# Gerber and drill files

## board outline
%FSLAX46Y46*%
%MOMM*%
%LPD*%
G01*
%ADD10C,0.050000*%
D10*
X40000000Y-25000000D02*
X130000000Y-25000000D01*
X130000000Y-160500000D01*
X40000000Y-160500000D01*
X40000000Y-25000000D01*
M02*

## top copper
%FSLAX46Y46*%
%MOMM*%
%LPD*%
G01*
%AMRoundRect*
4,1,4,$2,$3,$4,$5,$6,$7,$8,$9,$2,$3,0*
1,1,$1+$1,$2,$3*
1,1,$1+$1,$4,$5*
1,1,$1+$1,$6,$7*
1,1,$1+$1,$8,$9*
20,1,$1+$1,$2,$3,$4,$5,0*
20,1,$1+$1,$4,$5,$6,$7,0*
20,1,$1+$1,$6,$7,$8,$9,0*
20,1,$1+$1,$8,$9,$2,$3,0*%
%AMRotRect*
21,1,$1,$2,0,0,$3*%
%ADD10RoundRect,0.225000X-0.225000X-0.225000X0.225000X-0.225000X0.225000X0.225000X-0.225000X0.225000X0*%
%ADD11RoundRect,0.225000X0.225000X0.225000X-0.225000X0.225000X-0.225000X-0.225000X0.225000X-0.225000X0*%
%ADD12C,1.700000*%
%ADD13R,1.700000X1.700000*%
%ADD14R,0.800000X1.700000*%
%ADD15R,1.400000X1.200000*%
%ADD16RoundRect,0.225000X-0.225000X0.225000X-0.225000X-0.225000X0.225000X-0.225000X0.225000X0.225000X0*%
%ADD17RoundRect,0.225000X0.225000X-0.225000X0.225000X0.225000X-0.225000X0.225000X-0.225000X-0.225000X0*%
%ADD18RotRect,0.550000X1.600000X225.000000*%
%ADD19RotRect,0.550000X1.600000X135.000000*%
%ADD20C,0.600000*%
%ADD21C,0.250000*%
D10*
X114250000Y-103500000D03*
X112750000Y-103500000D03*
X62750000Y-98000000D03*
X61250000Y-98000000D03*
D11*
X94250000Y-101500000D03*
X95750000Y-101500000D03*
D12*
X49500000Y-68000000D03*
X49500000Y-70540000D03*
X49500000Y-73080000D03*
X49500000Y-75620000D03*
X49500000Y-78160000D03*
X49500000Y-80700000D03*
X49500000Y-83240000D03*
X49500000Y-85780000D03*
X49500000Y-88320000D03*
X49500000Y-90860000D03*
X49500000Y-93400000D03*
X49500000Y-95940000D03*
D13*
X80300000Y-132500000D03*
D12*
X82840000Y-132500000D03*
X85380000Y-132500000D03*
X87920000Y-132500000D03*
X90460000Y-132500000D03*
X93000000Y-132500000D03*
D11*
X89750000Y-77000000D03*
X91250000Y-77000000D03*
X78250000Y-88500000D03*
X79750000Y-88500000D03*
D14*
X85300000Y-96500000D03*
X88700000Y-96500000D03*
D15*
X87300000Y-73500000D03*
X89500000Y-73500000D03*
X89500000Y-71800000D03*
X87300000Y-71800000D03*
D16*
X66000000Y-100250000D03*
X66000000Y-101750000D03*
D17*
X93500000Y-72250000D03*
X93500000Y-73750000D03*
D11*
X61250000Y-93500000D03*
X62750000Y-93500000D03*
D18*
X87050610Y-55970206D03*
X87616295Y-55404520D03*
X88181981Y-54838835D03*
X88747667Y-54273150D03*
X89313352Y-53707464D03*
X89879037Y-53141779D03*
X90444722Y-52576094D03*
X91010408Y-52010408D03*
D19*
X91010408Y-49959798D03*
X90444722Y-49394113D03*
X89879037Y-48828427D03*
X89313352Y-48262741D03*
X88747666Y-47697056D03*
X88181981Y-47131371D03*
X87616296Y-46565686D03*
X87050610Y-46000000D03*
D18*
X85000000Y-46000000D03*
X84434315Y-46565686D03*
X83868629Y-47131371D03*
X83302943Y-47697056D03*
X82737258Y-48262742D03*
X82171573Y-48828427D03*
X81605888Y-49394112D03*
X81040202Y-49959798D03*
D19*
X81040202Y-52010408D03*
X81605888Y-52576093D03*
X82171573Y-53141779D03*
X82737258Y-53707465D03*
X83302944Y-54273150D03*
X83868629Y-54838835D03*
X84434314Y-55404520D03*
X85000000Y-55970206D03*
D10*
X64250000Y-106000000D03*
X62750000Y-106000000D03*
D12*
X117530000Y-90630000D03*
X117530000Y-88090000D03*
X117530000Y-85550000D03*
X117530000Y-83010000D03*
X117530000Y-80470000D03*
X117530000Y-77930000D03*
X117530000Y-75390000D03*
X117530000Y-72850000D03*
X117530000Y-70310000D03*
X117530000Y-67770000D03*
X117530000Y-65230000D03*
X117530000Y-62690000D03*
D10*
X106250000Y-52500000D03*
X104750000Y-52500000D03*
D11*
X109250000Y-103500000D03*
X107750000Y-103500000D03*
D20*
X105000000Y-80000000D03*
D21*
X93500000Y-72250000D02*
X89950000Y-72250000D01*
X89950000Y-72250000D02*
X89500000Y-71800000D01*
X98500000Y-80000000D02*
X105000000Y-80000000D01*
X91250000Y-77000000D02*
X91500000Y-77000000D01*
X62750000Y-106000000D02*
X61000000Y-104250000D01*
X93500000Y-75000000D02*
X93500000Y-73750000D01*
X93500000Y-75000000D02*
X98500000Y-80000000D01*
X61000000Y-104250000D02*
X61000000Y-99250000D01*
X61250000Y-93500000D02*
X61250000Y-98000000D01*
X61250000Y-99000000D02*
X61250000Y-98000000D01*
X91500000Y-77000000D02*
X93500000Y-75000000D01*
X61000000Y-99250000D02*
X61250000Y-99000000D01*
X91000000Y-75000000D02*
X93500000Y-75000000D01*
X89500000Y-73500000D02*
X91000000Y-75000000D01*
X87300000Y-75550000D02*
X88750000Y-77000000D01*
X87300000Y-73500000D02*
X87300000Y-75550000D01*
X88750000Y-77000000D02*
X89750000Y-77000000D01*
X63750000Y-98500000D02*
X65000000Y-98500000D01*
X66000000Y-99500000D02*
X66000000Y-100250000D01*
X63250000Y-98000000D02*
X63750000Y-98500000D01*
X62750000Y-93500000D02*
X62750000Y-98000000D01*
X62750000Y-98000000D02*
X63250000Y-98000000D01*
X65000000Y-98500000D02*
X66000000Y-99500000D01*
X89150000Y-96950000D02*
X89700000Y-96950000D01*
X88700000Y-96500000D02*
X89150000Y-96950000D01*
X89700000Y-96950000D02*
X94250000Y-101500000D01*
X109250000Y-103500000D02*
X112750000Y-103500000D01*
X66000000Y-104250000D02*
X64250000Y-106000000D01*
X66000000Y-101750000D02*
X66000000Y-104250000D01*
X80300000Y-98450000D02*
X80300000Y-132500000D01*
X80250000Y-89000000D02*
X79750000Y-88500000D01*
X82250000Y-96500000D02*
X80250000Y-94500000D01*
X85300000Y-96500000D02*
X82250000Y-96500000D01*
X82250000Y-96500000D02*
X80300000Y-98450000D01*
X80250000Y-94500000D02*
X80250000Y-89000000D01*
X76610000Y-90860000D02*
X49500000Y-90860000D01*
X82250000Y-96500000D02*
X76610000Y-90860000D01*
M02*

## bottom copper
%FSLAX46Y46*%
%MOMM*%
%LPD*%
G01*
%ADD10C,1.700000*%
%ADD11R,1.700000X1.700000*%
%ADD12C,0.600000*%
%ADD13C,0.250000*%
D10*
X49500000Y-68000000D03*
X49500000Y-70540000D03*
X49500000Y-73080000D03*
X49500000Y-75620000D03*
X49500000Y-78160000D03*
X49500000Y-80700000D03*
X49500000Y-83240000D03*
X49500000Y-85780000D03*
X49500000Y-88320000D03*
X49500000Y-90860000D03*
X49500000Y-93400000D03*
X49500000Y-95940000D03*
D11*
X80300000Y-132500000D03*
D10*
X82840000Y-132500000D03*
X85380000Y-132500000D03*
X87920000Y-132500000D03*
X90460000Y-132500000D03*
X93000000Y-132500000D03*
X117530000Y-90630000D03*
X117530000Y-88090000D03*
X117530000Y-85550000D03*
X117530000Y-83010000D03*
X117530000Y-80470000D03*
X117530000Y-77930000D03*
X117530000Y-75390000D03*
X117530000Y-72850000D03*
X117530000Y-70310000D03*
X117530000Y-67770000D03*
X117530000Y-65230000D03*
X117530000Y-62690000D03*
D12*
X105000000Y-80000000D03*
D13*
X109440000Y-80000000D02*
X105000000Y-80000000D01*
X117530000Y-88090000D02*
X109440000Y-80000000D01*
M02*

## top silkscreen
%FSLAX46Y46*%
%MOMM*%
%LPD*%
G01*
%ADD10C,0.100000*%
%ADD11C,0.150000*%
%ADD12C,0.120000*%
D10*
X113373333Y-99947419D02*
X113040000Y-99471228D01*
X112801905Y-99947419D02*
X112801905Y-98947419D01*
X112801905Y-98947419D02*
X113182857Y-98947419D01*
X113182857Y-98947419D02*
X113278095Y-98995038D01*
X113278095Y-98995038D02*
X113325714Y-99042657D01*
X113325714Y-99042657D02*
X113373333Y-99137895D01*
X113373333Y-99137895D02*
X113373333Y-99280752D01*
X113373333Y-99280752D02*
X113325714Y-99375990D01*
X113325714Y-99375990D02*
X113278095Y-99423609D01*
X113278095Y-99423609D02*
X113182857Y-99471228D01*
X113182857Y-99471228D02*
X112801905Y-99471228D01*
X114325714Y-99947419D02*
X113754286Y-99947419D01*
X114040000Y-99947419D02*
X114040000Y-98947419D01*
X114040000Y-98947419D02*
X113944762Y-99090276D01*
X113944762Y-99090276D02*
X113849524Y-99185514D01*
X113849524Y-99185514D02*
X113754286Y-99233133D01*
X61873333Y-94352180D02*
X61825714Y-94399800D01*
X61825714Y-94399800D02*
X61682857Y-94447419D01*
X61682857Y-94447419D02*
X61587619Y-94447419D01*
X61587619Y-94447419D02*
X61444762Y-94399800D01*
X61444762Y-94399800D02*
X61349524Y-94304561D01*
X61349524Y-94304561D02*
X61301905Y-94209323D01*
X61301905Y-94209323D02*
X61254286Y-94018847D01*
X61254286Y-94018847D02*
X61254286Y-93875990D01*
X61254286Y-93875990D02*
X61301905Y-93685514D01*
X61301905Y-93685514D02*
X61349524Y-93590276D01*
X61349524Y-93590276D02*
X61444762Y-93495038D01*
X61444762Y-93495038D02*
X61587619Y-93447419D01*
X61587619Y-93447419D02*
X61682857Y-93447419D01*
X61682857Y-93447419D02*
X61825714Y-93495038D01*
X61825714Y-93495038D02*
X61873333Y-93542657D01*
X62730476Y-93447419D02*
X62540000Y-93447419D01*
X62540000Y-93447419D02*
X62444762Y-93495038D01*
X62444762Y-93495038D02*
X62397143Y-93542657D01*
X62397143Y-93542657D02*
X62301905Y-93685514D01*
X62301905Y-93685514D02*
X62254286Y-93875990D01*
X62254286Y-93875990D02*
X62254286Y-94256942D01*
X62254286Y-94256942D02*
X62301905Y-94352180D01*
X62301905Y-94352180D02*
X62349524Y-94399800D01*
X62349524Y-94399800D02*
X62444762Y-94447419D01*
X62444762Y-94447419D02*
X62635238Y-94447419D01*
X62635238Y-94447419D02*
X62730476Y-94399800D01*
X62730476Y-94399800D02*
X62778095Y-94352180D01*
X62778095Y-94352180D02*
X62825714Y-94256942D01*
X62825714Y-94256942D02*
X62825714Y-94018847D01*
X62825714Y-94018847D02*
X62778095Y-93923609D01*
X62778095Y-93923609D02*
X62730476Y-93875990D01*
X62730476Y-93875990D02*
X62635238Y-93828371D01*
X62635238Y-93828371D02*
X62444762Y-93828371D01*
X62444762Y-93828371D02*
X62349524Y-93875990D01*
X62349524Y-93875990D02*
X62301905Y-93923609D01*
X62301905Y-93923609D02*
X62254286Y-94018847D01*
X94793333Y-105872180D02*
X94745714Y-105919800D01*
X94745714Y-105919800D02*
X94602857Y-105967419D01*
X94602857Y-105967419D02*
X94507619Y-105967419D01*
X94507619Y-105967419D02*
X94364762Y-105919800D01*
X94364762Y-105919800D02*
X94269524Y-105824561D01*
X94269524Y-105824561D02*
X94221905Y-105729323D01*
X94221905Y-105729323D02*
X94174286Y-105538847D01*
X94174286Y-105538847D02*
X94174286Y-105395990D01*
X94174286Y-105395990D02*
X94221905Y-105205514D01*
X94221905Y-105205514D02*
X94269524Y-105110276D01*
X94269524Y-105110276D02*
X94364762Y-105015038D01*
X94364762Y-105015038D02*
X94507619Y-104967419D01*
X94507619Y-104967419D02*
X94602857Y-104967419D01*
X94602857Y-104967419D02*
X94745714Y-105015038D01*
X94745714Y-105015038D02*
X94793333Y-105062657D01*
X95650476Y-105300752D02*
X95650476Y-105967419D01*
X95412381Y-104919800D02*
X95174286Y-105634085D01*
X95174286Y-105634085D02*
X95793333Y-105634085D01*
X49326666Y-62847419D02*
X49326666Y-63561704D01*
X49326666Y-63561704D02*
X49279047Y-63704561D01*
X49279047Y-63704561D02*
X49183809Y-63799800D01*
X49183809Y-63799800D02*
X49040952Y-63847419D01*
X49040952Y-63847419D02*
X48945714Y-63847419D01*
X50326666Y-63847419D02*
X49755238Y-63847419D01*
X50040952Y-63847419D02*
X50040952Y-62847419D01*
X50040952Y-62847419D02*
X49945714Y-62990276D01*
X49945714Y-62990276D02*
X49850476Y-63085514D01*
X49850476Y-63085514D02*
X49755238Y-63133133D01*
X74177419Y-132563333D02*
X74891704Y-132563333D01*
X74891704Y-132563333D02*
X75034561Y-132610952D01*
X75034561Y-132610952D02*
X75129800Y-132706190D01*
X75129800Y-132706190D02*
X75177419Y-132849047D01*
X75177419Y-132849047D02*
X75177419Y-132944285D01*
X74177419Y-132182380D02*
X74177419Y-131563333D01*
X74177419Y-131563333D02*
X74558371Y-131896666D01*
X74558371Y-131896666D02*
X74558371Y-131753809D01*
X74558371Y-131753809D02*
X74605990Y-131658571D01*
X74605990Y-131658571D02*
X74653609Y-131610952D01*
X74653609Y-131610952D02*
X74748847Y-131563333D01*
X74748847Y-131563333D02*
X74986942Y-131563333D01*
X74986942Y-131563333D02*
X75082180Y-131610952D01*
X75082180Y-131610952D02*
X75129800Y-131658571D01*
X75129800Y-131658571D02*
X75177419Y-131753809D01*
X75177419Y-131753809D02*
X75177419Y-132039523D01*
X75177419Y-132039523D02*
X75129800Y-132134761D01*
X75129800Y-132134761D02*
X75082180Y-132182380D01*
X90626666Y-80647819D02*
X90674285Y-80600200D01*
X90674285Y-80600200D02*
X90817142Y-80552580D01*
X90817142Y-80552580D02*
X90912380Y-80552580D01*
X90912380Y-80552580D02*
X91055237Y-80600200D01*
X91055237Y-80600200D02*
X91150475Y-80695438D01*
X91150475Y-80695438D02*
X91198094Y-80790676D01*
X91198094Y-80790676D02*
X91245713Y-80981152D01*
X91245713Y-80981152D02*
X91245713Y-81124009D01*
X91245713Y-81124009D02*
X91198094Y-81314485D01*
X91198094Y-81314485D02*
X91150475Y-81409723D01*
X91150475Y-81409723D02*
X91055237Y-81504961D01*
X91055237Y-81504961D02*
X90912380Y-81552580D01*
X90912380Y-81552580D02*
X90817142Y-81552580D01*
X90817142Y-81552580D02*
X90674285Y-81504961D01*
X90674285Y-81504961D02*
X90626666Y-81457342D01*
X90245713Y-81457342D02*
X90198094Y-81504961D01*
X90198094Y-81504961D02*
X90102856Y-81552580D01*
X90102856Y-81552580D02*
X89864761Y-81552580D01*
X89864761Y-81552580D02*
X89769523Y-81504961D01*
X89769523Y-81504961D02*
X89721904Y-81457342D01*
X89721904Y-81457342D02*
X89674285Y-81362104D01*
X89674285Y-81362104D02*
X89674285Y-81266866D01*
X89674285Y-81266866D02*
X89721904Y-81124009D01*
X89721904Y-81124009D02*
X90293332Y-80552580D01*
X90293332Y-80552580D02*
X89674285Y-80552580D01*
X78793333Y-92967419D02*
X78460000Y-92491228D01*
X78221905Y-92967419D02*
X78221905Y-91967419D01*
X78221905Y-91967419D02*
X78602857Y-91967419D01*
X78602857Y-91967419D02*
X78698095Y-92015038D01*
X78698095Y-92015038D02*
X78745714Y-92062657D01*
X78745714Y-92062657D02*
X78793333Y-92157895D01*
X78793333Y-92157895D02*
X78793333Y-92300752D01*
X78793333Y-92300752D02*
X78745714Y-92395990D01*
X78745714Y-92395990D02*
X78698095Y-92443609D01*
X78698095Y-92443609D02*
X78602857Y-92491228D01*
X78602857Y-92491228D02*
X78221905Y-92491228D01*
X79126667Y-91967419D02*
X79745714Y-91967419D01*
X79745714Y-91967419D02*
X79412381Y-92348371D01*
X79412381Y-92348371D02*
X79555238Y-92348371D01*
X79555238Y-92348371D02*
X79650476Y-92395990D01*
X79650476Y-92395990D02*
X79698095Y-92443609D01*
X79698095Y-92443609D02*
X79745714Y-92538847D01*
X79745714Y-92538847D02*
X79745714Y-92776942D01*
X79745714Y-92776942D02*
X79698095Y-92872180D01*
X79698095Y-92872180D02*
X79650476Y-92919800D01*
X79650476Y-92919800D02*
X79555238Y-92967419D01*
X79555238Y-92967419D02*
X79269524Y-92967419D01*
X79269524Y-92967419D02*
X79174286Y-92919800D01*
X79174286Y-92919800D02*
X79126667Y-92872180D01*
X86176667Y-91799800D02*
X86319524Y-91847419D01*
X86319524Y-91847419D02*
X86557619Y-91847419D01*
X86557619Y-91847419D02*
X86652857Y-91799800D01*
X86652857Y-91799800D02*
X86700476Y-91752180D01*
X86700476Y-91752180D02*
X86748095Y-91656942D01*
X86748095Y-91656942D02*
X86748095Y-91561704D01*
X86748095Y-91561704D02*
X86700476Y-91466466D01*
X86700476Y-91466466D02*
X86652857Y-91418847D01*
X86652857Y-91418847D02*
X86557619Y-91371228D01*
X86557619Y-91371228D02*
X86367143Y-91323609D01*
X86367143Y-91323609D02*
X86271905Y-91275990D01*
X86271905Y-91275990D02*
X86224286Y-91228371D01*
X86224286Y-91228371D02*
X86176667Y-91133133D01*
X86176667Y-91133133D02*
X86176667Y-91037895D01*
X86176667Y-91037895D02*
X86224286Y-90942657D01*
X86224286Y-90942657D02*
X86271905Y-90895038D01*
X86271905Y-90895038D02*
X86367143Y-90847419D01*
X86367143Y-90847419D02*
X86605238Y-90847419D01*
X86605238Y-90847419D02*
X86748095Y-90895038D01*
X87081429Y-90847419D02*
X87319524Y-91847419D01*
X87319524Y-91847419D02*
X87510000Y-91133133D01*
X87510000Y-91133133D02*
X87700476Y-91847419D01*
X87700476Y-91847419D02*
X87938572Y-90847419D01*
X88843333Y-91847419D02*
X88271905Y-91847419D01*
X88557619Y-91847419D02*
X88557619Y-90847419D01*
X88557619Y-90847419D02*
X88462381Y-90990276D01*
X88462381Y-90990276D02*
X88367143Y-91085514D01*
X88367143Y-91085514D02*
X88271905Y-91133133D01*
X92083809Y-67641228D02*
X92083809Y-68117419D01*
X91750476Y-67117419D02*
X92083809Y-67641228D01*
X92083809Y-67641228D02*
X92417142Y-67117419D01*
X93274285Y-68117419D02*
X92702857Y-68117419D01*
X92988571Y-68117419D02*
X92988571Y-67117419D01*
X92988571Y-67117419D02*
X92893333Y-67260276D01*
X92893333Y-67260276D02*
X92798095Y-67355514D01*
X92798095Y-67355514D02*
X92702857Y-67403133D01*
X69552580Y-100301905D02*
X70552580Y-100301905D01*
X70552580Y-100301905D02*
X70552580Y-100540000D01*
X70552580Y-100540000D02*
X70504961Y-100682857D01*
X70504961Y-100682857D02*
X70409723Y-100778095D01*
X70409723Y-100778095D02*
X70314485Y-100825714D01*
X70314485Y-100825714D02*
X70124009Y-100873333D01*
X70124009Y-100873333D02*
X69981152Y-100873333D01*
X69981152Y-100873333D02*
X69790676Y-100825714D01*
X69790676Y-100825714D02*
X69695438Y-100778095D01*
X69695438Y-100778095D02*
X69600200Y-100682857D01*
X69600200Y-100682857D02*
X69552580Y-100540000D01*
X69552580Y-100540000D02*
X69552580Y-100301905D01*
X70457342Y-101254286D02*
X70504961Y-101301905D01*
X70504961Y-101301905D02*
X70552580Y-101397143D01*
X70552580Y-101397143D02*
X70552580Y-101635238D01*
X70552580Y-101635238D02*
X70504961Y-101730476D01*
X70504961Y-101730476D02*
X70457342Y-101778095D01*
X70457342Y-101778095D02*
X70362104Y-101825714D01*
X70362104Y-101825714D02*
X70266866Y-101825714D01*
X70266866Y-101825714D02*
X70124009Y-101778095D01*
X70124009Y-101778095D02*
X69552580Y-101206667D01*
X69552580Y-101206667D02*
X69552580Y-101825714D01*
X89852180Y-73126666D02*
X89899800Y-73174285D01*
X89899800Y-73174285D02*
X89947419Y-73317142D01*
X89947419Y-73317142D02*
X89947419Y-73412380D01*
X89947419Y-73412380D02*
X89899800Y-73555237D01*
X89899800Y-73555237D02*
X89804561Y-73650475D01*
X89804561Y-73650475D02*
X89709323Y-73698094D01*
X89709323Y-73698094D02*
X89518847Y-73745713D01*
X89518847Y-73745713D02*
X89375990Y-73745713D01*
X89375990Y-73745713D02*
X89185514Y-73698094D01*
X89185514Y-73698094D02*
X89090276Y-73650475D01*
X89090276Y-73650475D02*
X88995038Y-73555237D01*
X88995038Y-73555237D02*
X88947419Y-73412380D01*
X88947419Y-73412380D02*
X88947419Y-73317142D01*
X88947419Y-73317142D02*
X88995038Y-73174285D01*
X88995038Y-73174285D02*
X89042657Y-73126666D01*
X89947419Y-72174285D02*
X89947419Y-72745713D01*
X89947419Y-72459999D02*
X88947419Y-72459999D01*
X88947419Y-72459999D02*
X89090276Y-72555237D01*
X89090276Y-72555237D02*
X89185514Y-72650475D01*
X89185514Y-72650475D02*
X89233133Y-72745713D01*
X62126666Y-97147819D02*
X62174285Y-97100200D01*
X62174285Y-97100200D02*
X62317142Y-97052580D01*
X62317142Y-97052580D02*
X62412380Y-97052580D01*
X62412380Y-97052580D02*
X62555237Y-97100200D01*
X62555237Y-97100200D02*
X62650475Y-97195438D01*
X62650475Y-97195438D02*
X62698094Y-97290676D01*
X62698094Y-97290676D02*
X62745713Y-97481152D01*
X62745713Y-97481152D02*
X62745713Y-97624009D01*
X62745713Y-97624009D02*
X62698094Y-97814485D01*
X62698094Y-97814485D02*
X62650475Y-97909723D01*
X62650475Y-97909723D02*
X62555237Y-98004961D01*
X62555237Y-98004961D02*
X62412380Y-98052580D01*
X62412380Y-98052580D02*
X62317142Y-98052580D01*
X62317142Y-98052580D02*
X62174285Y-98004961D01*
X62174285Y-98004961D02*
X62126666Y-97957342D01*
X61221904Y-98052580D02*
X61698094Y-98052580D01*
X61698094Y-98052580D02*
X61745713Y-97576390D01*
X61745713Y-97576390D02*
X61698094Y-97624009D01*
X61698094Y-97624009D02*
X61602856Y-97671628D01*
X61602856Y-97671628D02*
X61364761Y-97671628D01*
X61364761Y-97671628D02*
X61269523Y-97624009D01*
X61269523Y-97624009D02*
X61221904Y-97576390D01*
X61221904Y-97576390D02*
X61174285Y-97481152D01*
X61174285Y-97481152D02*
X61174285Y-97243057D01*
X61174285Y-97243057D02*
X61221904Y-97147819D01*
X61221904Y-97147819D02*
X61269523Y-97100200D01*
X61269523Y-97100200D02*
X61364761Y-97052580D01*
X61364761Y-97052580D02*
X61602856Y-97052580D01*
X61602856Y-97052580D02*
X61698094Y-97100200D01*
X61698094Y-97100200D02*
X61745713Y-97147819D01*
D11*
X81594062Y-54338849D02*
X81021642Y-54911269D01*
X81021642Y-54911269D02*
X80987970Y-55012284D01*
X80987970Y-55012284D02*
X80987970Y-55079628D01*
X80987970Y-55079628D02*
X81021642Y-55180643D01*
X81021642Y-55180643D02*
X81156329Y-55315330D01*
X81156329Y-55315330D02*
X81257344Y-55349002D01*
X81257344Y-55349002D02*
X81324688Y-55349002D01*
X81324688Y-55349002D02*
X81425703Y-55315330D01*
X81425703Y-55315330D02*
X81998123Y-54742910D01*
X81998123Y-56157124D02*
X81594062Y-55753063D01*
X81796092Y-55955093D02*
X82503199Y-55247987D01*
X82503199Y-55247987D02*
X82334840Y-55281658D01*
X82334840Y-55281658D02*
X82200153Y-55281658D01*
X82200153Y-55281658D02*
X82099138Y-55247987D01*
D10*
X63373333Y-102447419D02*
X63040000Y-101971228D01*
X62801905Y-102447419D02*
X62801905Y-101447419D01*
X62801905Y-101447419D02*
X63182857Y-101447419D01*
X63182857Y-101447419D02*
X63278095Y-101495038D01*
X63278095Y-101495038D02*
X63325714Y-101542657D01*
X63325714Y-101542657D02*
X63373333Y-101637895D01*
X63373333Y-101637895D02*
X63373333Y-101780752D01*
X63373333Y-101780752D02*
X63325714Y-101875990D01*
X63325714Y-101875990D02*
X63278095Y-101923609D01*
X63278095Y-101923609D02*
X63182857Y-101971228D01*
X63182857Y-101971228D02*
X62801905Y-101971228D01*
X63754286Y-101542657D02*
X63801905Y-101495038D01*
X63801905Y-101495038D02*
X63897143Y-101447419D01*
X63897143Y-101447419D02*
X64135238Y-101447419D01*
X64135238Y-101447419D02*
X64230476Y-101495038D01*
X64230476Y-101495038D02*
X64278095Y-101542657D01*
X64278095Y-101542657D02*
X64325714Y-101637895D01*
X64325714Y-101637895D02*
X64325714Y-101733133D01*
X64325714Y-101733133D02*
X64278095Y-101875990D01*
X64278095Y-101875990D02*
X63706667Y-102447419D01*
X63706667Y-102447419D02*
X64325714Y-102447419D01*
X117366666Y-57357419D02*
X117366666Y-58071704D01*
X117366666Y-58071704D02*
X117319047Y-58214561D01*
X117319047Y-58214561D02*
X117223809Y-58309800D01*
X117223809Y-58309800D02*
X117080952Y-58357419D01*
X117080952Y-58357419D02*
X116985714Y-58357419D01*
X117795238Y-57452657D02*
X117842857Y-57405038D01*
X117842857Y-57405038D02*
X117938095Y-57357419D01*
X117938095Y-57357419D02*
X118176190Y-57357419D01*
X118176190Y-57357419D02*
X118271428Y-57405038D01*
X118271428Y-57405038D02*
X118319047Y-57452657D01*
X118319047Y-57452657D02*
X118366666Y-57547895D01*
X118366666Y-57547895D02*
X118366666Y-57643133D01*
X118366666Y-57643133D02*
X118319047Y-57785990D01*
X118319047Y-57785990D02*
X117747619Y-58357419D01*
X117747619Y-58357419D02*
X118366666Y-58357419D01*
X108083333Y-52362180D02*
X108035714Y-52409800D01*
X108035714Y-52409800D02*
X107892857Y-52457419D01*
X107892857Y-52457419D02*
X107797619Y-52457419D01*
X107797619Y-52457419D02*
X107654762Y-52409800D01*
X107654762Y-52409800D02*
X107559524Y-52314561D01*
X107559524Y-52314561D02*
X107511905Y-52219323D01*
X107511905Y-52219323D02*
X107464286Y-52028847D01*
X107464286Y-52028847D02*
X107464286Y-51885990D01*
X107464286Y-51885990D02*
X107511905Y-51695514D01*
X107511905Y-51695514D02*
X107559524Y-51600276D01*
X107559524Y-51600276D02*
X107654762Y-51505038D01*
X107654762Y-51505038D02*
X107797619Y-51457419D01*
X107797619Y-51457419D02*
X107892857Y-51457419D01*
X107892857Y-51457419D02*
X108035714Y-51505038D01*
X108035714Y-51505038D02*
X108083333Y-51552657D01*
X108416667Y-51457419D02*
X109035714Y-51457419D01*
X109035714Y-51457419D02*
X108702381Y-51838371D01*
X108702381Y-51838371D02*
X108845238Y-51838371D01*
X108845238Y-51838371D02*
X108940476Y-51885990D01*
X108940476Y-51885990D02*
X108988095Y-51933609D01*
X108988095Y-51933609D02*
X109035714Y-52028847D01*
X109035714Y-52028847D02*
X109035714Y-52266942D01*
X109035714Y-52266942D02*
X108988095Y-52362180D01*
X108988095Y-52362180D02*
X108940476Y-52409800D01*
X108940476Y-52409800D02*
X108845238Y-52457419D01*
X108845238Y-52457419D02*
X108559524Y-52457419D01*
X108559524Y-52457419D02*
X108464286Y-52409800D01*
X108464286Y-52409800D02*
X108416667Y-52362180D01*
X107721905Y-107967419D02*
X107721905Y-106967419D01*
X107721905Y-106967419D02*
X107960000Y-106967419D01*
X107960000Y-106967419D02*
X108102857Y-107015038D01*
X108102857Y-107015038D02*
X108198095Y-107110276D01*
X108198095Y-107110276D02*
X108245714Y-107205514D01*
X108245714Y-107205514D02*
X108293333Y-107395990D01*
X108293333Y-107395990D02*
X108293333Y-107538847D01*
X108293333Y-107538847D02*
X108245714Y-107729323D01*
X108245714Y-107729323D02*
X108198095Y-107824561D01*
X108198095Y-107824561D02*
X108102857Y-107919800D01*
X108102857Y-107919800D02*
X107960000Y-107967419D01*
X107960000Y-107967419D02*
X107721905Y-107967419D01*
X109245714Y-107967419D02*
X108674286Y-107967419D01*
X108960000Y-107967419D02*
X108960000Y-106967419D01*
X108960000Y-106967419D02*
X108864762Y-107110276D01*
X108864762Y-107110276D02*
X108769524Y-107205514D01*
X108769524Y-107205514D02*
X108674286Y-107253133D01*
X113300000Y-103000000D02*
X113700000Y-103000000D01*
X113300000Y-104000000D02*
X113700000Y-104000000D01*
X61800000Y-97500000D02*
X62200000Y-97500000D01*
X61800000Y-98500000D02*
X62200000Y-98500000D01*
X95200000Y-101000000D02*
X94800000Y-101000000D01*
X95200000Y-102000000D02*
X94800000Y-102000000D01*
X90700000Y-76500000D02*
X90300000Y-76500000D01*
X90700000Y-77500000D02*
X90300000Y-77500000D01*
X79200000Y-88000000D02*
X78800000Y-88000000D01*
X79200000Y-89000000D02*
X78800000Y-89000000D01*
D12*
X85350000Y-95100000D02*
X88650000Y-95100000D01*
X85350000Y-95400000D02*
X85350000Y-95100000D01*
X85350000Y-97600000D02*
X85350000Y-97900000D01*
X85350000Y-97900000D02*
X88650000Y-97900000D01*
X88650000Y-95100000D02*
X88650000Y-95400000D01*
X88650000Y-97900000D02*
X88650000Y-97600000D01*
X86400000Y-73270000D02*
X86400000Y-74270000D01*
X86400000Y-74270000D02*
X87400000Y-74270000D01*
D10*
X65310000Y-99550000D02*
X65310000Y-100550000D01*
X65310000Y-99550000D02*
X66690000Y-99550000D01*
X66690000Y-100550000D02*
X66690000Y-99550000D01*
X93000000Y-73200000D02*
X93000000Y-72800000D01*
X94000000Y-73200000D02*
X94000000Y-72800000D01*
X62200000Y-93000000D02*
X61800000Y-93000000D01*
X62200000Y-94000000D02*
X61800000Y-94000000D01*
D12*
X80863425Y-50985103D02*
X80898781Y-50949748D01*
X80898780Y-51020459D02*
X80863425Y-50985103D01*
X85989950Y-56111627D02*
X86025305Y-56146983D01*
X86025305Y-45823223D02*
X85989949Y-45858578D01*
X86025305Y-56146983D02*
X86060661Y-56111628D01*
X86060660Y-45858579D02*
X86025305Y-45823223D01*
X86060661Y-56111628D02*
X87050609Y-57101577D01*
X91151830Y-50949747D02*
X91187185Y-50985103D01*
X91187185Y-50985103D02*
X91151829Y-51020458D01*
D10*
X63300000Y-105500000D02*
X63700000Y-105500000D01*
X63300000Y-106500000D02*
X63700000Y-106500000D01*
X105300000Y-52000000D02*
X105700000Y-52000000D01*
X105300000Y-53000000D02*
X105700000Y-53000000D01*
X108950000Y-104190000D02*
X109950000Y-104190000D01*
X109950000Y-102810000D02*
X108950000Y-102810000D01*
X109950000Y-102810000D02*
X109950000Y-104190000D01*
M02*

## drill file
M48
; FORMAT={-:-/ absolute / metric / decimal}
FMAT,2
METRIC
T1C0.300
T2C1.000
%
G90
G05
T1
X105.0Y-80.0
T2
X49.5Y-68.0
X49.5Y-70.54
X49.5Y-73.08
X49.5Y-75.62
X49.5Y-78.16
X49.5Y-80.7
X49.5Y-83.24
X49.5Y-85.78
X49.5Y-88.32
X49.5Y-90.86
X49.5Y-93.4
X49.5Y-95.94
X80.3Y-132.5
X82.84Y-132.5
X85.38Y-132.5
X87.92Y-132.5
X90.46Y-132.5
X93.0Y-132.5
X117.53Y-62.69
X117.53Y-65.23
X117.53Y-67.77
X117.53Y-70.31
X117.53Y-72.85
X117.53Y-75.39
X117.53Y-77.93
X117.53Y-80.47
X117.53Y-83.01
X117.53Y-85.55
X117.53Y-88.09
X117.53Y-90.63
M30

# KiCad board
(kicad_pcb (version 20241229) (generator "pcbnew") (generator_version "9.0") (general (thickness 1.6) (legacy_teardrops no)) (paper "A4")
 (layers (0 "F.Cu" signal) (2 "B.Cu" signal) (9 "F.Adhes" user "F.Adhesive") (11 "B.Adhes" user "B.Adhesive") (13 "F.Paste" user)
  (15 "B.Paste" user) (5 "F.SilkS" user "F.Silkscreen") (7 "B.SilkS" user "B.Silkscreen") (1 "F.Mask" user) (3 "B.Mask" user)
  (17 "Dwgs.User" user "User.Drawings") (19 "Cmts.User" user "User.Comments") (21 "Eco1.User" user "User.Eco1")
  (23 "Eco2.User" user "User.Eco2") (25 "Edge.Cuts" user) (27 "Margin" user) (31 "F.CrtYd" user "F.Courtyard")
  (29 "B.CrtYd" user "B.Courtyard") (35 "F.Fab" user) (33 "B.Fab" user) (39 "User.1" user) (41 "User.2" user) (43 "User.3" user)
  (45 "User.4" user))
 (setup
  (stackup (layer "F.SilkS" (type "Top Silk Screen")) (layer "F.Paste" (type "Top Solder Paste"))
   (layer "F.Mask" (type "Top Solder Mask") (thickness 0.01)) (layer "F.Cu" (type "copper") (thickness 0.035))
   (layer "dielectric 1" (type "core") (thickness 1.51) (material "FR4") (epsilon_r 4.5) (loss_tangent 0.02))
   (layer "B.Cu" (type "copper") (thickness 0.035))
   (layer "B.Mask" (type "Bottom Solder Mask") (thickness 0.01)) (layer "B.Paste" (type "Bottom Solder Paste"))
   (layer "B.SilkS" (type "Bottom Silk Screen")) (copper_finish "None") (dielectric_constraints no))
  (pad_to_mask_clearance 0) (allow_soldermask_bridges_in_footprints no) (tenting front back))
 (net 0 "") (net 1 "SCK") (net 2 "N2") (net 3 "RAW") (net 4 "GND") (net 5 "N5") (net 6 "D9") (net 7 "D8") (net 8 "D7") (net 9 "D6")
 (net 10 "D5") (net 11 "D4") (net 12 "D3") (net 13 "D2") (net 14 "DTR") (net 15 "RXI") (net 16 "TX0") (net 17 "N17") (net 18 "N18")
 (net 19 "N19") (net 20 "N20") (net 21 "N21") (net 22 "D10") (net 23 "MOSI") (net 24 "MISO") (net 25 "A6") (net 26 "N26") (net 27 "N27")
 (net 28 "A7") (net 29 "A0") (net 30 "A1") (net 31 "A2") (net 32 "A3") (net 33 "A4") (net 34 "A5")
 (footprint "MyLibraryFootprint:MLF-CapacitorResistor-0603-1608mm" (layer "F.Cu") (at 113.5 103.5)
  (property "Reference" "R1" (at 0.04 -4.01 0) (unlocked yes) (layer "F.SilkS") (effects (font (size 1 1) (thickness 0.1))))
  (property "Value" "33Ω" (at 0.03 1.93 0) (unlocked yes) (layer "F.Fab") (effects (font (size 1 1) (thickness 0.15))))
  (fp_line (start -0.2 -0.5) (end 0.2 -0.5) (stroke (width 0.1) (type solid)) (layer "F.SilkS"))
  (fp_line (start -0.2 0.5) (end 0.2 0.5) (stroke (width 0.1) (type solid)) (layer "F.SilkS"))
  (pad "1" smd roundrect (at 0.75 0) (size 0.9 0.9) (layers "F.Cu" "F.Mask" "F.Paste") (roundrect_rratio 0.25) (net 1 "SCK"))
  (pad "2" smd roundrect (at -0.75 0) (size 0.9 0.9) (layers "F.Cu" "F.Mask" "F.Paste") (roundrect_rratio 0.25) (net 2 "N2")))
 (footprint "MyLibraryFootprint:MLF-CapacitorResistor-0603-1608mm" (layer "F.Cu") (at 62 98)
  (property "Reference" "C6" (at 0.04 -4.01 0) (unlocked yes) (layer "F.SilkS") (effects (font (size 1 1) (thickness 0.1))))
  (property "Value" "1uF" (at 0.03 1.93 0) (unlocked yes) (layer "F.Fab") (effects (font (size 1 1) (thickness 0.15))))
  (fp_line (start -0.2 -0.5) (end 0.2 -0.5) (stroke (width 0.1) (type solid)) (layer "F.SilkS"))
  (fp_line (start -0.2 0.5) (end 0.2 0.5) (stroke (width 0.1) (type solid)) (layer "F.SilkS"))
  (pad "1" smd roundrect (at 0.75 0) (size 0.9 0.9) (layers "F.Cu" "F.Mask" "F.Paste") (roundrect_rratio 0.25) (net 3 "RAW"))
  (pad "2" smd roundrect (at -0.75 0) (size 0.9 0.9) (layers "F.Cu" "F.Mask" "F.Paste") (roundrect_rratio 0.25) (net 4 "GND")))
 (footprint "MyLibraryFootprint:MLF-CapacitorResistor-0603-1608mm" (layer "F.Cu") (at 95 101.5 180)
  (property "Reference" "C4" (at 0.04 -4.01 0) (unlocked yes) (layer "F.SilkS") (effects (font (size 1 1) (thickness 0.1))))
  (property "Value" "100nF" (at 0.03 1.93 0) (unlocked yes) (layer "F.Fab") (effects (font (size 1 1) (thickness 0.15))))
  (fp_line (start -0.2 0.5) (end 0.2 0.5) (stroke (width 0.1) (type solid)) (layer "F.SilkS"))
  (fp_line (start -0.2 -0.5) (end 0.2 -0.5) (stroke (width 0.1) (type solid)) (layer "F.SilkS"))
  (pad "1" smd roundrect (at 0.75 0 180) (size 0.9 0.9) (layers "F.Cu" "F.Mask" "F.Paste") (roundrect_rratio 0.25) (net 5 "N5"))
  (pad "2" smd roundrect (at -0.75 0 180) (size 0.9 0.9) (layers "F.Cu" "F.Mask" "F.Paste") (roundrect_rratio 0.25) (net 4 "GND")))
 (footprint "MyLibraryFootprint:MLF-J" (layer "F.Cu") (at 49.71 73.61)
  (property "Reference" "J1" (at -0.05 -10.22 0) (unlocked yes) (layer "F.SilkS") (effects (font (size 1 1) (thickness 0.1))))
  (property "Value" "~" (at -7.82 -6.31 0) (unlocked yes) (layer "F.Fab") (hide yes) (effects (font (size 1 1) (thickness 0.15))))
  (pad "1" thru_hole circle (at -0.21 -5.61) (size 1.7 1.7) (drill 1) (layers "*.Cu" "*.Mask") (remove_unused_layers no) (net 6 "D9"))
  (pad "2" thru_hole circle (at -0.21 -3.07) (size 1.7 1.7) (drill 1) (layers "*.Cu" "*.Mask") (remove_unused_layers no) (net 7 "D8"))
  (pad "3" thru_hole circle (at -0.21 -0.53) (size 1.7 1.7) (drill 1) (layers "*.Cu" "*.Mask") (remove_unused_layers no) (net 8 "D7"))
  (pad "4" thru_hole circle (at -0.21 2.01) (size 1.7 1.7) (drill 1) (layers "*.Cu" "*.Mask") (remove_unused_layers no) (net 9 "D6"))
  (pad "5" thru_hole circle (at -0.21 4.55) (size 1.7 1.7) (drill 1) (layers "*.Cu" "*.Mask") (remove_unused_layers no) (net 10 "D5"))
  (pad "6" thru_hole circle (at -0.21 7.09) (size 1.7 1.7) (drill 1) (layers "*.Cu" "*.Mask") (remove_unused_layers no) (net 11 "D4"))
  (pad "7" thru_hole circle (at -0.21 9.63) (size 1.7 1.7) (drill 1) (layers "*.Cu" "*.Mask") (remove_unused_layers no) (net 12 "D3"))
  (pad "8" thru_hole circle (at -0.21 12.17) (size 1.7 1.7) (drill 1) (layers "*.Cu" "*.Mask") (remove_unused_layers no) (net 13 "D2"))
  (pad "9" thru_hole circle (at -0.21 14.71) (size 1.7 1.7) (drill 1) (layers "*.Cu" "*.Mask") (remove_unused_layers no) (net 4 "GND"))
  (pad "10" thru_hole circle (at -0.21 17.25) (size 1.7 1.7) (drill 1) (layers "*.Cu" "*.Mask") (remove_unused_layers no) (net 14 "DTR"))
  (pad "11" thru_hole circle (at -0.21 19.79) (size 1.7 1.7) (drill 1) (layers "*.Cu" "*.Mask") (remove_unused_layers no) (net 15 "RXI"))
  (pad "12" thru_hole circle (at -0.21 22.33) (size 1.7 1.7) (drill 1) (layers "*.Cu" "*.Mask") (remove_unused_layers no) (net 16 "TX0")))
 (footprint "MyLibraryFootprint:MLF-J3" (layer "F.Cu") (at 88.37 132.33 90)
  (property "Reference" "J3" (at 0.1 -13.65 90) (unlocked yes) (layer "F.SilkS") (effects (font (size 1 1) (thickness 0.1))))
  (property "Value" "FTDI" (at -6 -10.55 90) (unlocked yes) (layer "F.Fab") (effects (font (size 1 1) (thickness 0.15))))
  (pad "1" thru_hole rect (at -0.17 -8.07 90) (size 1.7 1.7) (drill 1) (layers "*.Cu" "*.Mask") (remove_unused_layers no) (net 14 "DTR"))
  (pad "2" thru_hole circle (at -0.17 -5.53 90) (size 1.7 1.7) (drill 1) (layers "*.Cu" "*.Mask") (remove_unused_layers no) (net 16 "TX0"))
  (pad "3" thru_hole circle (at -0.17 -2.99 90) (size 1.7 1.7) (drill 1) (layers "*.Cu" "*.Mask") (remove_unused_layers no) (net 15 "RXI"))
  (pad "4" thru_hole circle (at -0.17 -0.45 90) (size 1.7 1.7) (drill 1) (layers "*.Cu" "*.Mask") (remove_unused_layers no) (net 3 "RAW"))
  (pad "5" thru_hole circle (at -0.17 2.09 90) (size 1.7 1.7) (drill 1) (layers "*.Cu" "*.Mask") (remove_unused_layers no) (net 4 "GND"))
  (pad "6" thru_hole circle (at -0.17 4.63 90) (size 1.7 1.7) (drill 1) (layers "*.Cu" "*.Mask") (remove_unused_layers no) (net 4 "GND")))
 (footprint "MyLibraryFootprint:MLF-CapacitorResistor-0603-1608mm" (layer "F.Cu") (at 90.5 77 180)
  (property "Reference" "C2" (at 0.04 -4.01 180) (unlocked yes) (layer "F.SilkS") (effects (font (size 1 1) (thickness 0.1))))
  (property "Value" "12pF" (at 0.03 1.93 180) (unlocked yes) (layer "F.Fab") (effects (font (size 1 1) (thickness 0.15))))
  (fp_line (start -0.2 0.5) (end 0.2 0.5) (stroke (width 0.1) (type solid)) (layer "F.SilkS"))
  (fp_line (start -0.2 -0.5) (end 0.2 -0.5) (stroke (width 0.1) (type solid)) (layer "F.SilkS"))
  (pad "1" smd roundrect (at 0.75 0 180) (size 0.9 0.9) (layers "F.Cu" "F.Mask" "F.Paste") (roundrect_rratio 0.25) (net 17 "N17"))
  (pad "2" smd roundrect (at -0.75 0 180) (size 0.9 0.9) (layers "F.Cu" "F.Mask" "F.Paste") (roundrect_rratio 0.25) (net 4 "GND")))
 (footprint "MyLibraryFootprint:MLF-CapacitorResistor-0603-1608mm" (layer "F.Cu") (at 79 88.5 180)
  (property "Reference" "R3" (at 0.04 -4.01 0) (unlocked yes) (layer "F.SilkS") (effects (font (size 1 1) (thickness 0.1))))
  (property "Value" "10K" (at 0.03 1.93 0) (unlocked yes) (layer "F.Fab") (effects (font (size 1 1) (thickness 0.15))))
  (fp_line (start -0.2 0.5) (end 0.2 0.5) (stroke (width 0.1) (type solid)) (layer "F.SilkS"))
  (fp_line (start -0.2 -0.5) (end 0.2 -0.5) (stroke (width 0.1) (type solid)) (layer "F.SilkS"))
  (pad "1" smd roundrect (at 0.75 0 180) (size 0.9 0.9) (layers "F.Cu" "F.Mask" "F.Paste") (roundrect_rratio 0.25) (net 3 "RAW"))
  (pad "2" smd roundrect (at -0.75 0 180) (size 0.9 0.9) (layers "F.Cu" "F.Mask" "F.Paste") (roundrect_rratio 0.25) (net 14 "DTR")))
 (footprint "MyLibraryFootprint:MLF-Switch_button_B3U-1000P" (layer "F.Cu") (at 87 96.5)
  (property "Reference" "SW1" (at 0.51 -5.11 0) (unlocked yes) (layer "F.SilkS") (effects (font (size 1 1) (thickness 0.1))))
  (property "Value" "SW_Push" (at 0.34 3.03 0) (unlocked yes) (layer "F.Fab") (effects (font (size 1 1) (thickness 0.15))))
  (fp_line (start -1.65 -1.4) (end 1.65 -1.4) (stroke (width 0.12) (type solid)) (layer "F.SilkS"))
  (fp_line (start -1.65 -1.1) (end -1.65 -1.4) (stroke (width 0.12) (type solid)) (layer "F.SilkS"))
  (fp_line (start -1.65 1.1) (end -1.65 1.4) (stroke (width 0.12) (type solid)) (layer "F.SilkS"))
  (fp_line (start -1.65 1.4) (end 1.65 1.4) (stroke (width 0.12) (type solid)) (layer "F.SilkS"))
  (fp_line (start 1.65 -1.4) (end 1.65 -1.1) (stroke (width 0.12) (type solid)) (layer "F.SilkS"))
  (fp_line (start 1.65 1.4) (end 1.65 1.1) (stroke (width 0.12) (type solid)) (layer "F.SilkS"))
  (pad "1" smd rect (at -1.7 0) (size 0.8 1.7) (layers "F.Cu" "F.Mask" "F.Paste") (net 14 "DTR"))
  (pad "2" smd rect (at 1.7 0) (size 0.8 1.7) (layers "F.Cu" "F.Mask" "F.Paste") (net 5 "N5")))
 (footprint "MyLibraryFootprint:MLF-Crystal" (layer "F.Cu") (at 88.38 72.61)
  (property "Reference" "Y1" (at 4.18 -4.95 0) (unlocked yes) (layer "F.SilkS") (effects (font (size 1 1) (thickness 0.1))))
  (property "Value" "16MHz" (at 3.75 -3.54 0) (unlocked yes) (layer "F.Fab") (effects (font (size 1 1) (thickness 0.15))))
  (fp_line (start -1.98 0.66) (end -1.98 1.66) (stroke (width 0.12) (type solid)) (layer "F.SilkS"))
  (fp_line (start -1.98 1.66) (end -0.98 1.66) (stroke (width 0.12) (type solid)) (layer "F.SilkS"))
  (pad "1" smd rect (at -1.08 0.89) (size 1.4 1.2) (layers "F.Cu" "F.Mask" "F.Paste") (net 17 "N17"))
  (pad "2" smd rect (at 1.12 0.89) (size 1.4 1.2) (layers "F.Cu" "F.Mask" "F.Paste") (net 4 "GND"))
  (pad "3" smd rect (at 1.12 -0.81) (size 1.4 1.2) (layers "F.Cu" "F.Mask" "F.Paste") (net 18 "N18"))
  (pad "4" smd rect (at -1.08 -0.81) (size 1.4 1.2) (layers "F.Cu" "F.Mask" "F.Paste") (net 4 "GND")))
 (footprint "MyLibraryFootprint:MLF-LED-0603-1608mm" (layer "F.Cu") (at 66 101 -90)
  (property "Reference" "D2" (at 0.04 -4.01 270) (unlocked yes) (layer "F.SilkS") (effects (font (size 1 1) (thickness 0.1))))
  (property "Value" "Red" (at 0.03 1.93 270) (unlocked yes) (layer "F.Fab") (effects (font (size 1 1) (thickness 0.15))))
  (fp_line (start -1.45 0.69) (end -0.45 0.69) (stroke (width 0.1) (type solid)) (layer "F.SilkS"))
  (fp_line (start -1.45 0.69) (end -1.45 -0.69) (stroke (width 0.1) (type default)) (layer "F.SilkS"))
  (fp_line (start -0.45 -0.69) (end -1.45 -0.69) (stroke (width 0.1) (type solid)) (layer "F.SilkS"))
  (pad "1" smd roundrect (at -0.75 0 270) (size 0.9 0.9) (layers "F.Cu" "F.Mask" "F.Paste") (roundrect_rratio 0.25) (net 3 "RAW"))
  (pad "2" smd roundrect (at 0.75 0 270) (size 0.9 0.9) (layers "F.Cu" "F.Mask" "F.Paste") (roundrect_rratio 0.25) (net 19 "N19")))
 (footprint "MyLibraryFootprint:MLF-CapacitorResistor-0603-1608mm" (layer "F.Cu") (at 93.5 73 90)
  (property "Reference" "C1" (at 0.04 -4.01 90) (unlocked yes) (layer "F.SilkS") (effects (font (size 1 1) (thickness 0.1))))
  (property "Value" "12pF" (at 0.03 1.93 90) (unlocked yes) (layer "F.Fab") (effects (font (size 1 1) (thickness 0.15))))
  (fp_line (start -0.2 -0.5) (end 0.2 -0.5) (stroke (width 0.1) (type solid)) (layer "F.SilkS"))
  (fp_line (start -0.2 0.5) (end 0.2 0.5) (stroke (width 0.1) (type solid)) (layer "F.SilkS"))
  (pad "1" smd roundrect (at 0.75 0 90) (size 0.9 0.9) (layers "F.Cu" "F.Mask" "F.Paste") (roundrect_rratio 0.25) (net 18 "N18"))
  (pad "2" smd roundrect (at -0.75 0 90) (size 0.9 0.9) (layers "F.Cu" "F.Mask" "F.Paste") (roundrect_rratio 0.25) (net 4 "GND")))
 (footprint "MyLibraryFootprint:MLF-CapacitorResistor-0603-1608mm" (layer "F.Cu") (at 62 93.5 180)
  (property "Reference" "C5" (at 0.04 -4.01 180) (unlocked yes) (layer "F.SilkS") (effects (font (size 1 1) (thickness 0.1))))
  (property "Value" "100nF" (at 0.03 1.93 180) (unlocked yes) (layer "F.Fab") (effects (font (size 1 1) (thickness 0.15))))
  (fp_line (start -0.2 0.5) (end 0.2 0.5) (stroke (width 0.1) (type solid)) (layer "F.SilkS"))
  (fp_line (start -0.2 -0.5) (end 0.2 -0.5) (stroke (width 0.1) (type solid)) (layer "F.SilkS"))
  (pad "1" smd roundrect (at 0.75 0 180) (size 0.9 0.9) (layers "F.Cu" "F.Mask" "F.Paste") (roundrect_rratio 0.25) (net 4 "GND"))
  (pad "2" smd roundrect (at -0.75 0 180) (size 0.9 0.9) (layers "F.Cu" "F.Mask" "F.Paste") (roundrect_rratio 0.25) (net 3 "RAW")))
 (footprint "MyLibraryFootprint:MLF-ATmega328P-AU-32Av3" (layer "F.Cu") (at 86.025305 50.985103 135)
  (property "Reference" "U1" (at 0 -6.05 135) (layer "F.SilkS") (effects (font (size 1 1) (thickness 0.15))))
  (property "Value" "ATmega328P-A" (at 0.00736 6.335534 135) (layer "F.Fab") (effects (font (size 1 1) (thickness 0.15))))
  (fp_line (start 3.65 -3.65) (end 3.65 -3.6) (stroke (width 0.12) (type default)) (layer "F.SilkS"))
  (fp_line (start 3.6 -3.650001) (end 3.65 -3.65) (stroke (width 0.12) (type default)) (layer "F.SilkS"))
  (fp_line (start -3.6 -3.65) (end -3.65 -3.65) (stroke (width 0.12) (type default)) (layer "F.SilkS"))
  (fp_line (start 3.65 3.65) (end 3.650001 3.6) (stroke (width 0.12) (type default)) (layer "F.SilkS"))
  (fp_line (start -3.65 -3.65) (end -3.650001 -3.6) (stroke (width 0.12) (type default)) (layer "F.SilkS"))
  (fp_line (start 3.6 3.65) (end 3.65 3.65) (stroke (width 0.12) (type default)) (layer "F.SilkS"))
  (fp_line (start -3.650001 -3.6) (end -5.05 -3.600001) (stroke (width 0.12) (type default)) (layer "F.SilkS"))
  (fp_line (start -3.6 3.650001) (end -3.65 3.65) (stroke (width 0.12) (type default)) (layer "F.SilkS"))
  (fp_line (start -3.65 3.65) (end -3.65 3.6) (stroke (width 0.12) (type default)) (layer "F.SilkS"))
  (pad "1" smd rect (at -4.25 -2.8 225) (size 0.55 1.6) (layers "F.Cu" "F.Mask" "F.Paste") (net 12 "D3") (thermal_bridge_angle 45))
  (pad "2" smd rect (at -4.25 -2 225) (size 0.55 1.6) (layers "F.Cu" "F.Mask" "F.Paste") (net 11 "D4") (thermal_bridge_angle 45))
  (pad "3" smd rect (at -4.25 -1.2 225) (size 0.55 1.6) (layers "F.Cu" "F.Mask" "F.Paste") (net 4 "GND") (thermal_bridge_angle 45))
  (pad "4" smd rect (at -4.250001 -0.4 225) (size 0.55 1.6) (layers "F.Cu" "F.Mask" "F.Paste") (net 3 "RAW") (thermal_bridge_angle 45))
  (pad "5" smd rect (at -4.25 0.4 225) (size 0.55 1.6) (layers "F.Cu" "F.Mask" "F.Paste") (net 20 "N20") (thermal_bridge_angle 45))
  (pad "6" smd rect (at -4.25 1.2 225) (size 0.55 1.6) (layers "F.Cu" "F.Mask" "F.Paste") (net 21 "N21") (thermal_bridge_angle 45))
  (pad "7" smd rect (at -4.25 1.999999 225) (size 0.55 1.6) (layers "F.Cu" "F.Mask" "F.Paste") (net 17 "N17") (thermal_bridge_angle 45))
  (pad "8" smd rect (at -4.25 2.8 225) (size 0.55 1.6) (layers "F.Cu" "F.Mask" "F.Paste") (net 18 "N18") (thermal_bridge_angle 45))
  (pad "9" smd rect (at -2.8 4.25 135) (size 0.55 1.6) (layers "F.Cu" "F.Mask" "F.Paste") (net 10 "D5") (thermal_bridge_angle 45))
  (pad "10" smd rect (at -2 4.25 135) (size 0.55 1.6) (layers "F.Cu" "F.Mask" "F.Paste") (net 9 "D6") (thermal_bridge_angle 45))
  (pad "11" smd rect (at -1.2 4.25 135) (size 0.55 1.6) (layers "F.Cu" "F.Mask" "F.Paste") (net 8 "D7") (thermal_bridge_angle 45))
  (pad "12" smd rect (at -0.4 4.250001 135) (size 0.55 1.6) (layers "F.Cu" "F.Mask" "F.Paste") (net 7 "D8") (thermal_bridge_angle 45))
  (pad "13" smd rect (at 0.4 4.25 135) (size 0.55 1.6) (layers "F.Cu" "F.Mask" "F.Paste") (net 6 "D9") (thermal_bridge_angle 45))
  (pad "14" smd rect (at 1.2 4.25 135) (size 0.55 1.6) (layers "F.Cu" "F.Mask" "F.Paste") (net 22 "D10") (thermal_bridge_angle 45))
  (pad "15" smd rect (at 1.999999 4.25 135) (size 0.55 1.6) (layers "F.Cu" "F.Mask" "F.Paste") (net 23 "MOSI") (thermal_bridge_angle 45))
  (pad "16" smd rect (at 2.8 4.25 135) (size 0.55 1.6) (layers "F.Cu" "F.Mask" "F.Paste") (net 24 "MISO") (thermal_bridge_angle 45))
  (pad "17" smd rect (at 4.25 2.8 225) (size 0.55 1.6) (layers "F.Cu" "F.Mask" "F.Paste") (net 1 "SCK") (thermal_bridge_angle 45))
  (pad "18" smd rect (at 4.25 2 225) (size 0.55 1.6) (layers "F.Cu" "F.Mask" "F.Paste") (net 3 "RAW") (thermal_bridge_angle 45))
  (pad "19" smd rect (at 4.25 1.2 225) (size 0.55 1.6) (layers "F.Cu" "F.Mask" "F.Paste") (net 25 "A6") (thermal_bridge_angle 45))
  (pad "20" smd rect (at 4.250001 0.4 225) (size 0.55 1.6) (layers "F.Cu" "F.Mask" "F.Paste") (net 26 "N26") (thermal_bridge_angle 45))
  (pad "21" smd rect (at 4.25 -0.4 225) (size 0.55 1.6) (layers "F.Cu" "F.Mask" "F.Paste") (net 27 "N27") (thermal_bridge_angle 45))
  (pad "22" smd rect (at 4.25 -1.2 225) (size 0.55 1.6) (layers "F.Cu" "F.Mask" "F.Paste") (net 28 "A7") (thermal_bridge_angle 45))
  (pad "23" smd rect (at 4.25 -1.999999 225) (size 0.55 1.6) (layers "F.Cu" "F.Mask" "F.Paste") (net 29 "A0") (thermal_bridge_angle 45))
  (pad "24" smd rect (at 4.25 -2.8 225) (size 0.55 1.6) (layers "F.Cu" "F.Mask" "F.Paste") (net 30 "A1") (thermal_bridge_angle 45))
  (pad "25" smd rect (at 2.8 -4.25 135) (size 0.55 1.6) (layers "F.Cu" "F.Mask" "F.Paste") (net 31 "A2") (thermal_bridge_angle 45))
  (pad "26" smd rect (at 2 -4.25 135) (size 0.55 1.6) (layers "F.Cu" "F.Mask" "F.Paste") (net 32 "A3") (thermal_bridge_angle 45))
  (pad "27" smd rect (at 1.2 -4.25 135) (size 0.55 1.6) (layers "F.Cu" "F.Mask" "F.Paste") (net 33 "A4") (thermal_bridge_angle 45))
  (pad "28" smd rect (at 0.4 -4.250001 135) (size 0.55 1.6) (layers "F.Cu" "F.Mask" "F.Paste") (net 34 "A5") (thermal_bridge_angle 45))
  (pad "29" smd rect (at -0.4 -4.25 135) (size 0.55 1.6) (layers "F.Cu" "F.Mask" "F.Paste") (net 14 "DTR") (thermal_bridge_angle 45))
  (pad "30" smd rect (at -1.2 -4.25 135) (size 0.55 1.6) (layers "F.Cu" "F.Mask" "F.Paste") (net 15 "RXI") (thermal_bridge_angle 45))
  (pad "31" smd rect (at -1.999999 -4.25 135) (size 0.55 1.6) (layers "F.Cu" "F.Mask" "F.Paste") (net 16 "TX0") (thermal_bridge_angle 45))
  (pad "32" smd rect (at -2.8 -4.25 135) (size 0.55 1.6) (layers "F.Cu" "F.Mask" "F.Paste") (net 13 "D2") (thermal_bridge_angle 45)))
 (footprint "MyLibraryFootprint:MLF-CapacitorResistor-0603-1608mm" (layer "F.Cu") (at 63.5 106)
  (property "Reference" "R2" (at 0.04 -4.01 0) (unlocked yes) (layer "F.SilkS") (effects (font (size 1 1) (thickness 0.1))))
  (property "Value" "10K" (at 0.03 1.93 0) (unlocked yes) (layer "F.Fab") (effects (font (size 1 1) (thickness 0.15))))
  (fp_line (start -0.2 -0.5) (end 0.2 -0.5) (stroke (width 0.1) (type solid)) (layer "F.SilkS"))
  (fp_line (start -0.2 0.5) (end 0.2 0.5) (stroke (width 0.1) (type solid)) (layer "F.SilkS"))
  (pad "1" smd roundrect (at 0.75 0) (size 0.9 0.9) (layers "F.Cu" "F.Mask" "F.Paste") (roundrect_rratio 0.25) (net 19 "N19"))
  (pad "2" smd roundrect (at -0.75 0) (size 0.9 0.9) (layers "F.Cu" "F.Mask" "F.Paste") (roundrect_rratio 0.25) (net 4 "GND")))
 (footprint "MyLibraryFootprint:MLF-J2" (layer "F.Cu") (at 117.5 69.5)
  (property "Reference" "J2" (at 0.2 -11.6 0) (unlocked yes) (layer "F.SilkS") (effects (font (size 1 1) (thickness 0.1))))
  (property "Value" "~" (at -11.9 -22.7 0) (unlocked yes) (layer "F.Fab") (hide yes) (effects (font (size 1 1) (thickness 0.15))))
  (pad "1" thru_hole circle (at 0.03 21.13) (size 1.7 1.7) (drill 1) (layers "*.Cu" "*.Mask") (remove_unused_layers no) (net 3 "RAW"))
  (pad "2" thru_hole circle (at 0.03 18.59) (size 1.7 1.7) (drill 1) (layers "*.Cu" "*.Mask") (remove_unused_layers no) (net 4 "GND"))
  (pad "3" thru_hole circle (at 0.03 16.05) (size 1.7 1.7) (drill 1) (layers "*.Cu" "*.Mask") (remove_unused_layers no) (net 14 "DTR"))
  (pad "4" thru_hole circle (at 0.03 13.51) (size 1.7 1.7) (drill 1) (layers "*.Cu" "*.Mask") (remove_unused_layers no) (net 3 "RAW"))
  (pad "5" thru_hole circle (at 0.03 10.97) (size 1.7 1.7) (drill 1) (layers "*.Cu" "*.Mask") (remove_unused_layers no) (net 32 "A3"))
  (pad "6" thru_hole circle (at 0.03 8.43) (size 1.7 1.7) (drill 1) (layers "*.Cu" "*.Mask") (remove_unused_layers no) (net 31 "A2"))
  (pad "7" thru_hole circle (at 0.03 5.89) (size 1.7 1.7) (drill 1) (layers "*.Cu" "*.Mask") (remove_unused_layers no) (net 30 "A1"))
  (pad "8" thru_hole circle (at 0.03 3.35) (size 1.7 1.7) (drill 1) (layers "*.Cu" "*.Mask") (remove_unused_layers no) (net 29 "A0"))
  (pad "9" thru_hole circle (at 0.03 0.81) (size 1.7 1.7) (drill 1) (layers "*.Cu" "*.Mask") (remove_unused_layers no) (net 1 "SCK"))
  (pad "10" thru_hole circle (at 0.03 -1.73) (size 1.7 1.7) (drill 1) (layers "*.Cu" "*.Mask") (remove_unused_layers no) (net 24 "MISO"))
  (pad "11" thru_hole circle (at 0.03 -4.27) (size 1.7 1.7) (drill 1) (layers "*.Cu" "*.Mask") (remove_unused_layers no) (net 23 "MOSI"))
  (pad "12" thru_hole circle (at 0.03 -6.81) (size 1.7 1.7) (drill 1) (layers "*.Cu" "*.Mask") (remove_unused_layers no) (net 22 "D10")))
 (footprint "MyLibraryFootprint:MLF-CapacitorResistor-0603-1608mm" (layer "F.Cu") (at 105.5 52.5)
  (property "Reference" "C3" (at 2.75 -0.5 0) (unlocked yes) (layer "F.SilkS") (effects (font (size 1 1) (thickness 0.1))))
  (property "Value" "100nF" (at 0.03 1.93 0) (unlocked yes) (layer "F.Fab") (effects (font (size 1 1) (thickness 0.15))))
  (fp_line (start -0.2 -0.5) (end 0.2 -0.5) (stroke (width 0.1) (type solid)) (layer "F.SilkS"))
  (fp_line (start -0.2 0.5) (end 0.2 0.5) (stroke (width 0.1) (type solid)) (layer "F.SilkS"))
  (pad "1" smd roundrect (at 0.75 0) (size 0.9 0.9) (layers "F.Cu" "F.Mask" "F.Paste") (roundrect_rratio 0.25) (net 3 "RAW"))
  (pad "2" smd roundrect (at -0.75 0) (size 0.9 0.9) (layers "F.Cu" "F.Mask" "F.Paste") (roundrect_rratio 0.25) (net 26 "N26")))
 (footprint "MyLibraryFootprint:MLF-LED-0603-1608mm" (layer "F.Cu") (at 108.5 103.5 180)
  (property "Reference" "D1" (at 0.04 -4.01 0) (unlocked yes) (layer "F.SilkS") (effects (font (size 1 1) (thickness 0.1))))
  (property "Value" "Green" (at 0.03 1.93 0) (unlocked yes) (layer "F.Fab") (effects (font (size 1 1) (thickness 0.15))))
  (fp_line (start -0.45 -0.69) (end -1.45 -0.69) (stroke (width 0.1) (type solid)) (layer "F.SilkS"))
  (fp_line (start -1.45 0.69) (end -0.45 0.69) (stroke (width 0.1) (type solid)) (layer "F.SilkS"))
  (fp_line (start -1.45 0.69) (end -1.45 -0.69) (stroke (width 0.1) (type default)) (layer "F.SilkS"))
  (pad "1" smd roundrect (at -0.75 0 180) (size 0.9 0.9) (layers "F.Cu" "F.Mask" "F.Paste") (roundrect_rratio 0.25) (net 2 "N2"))
  (pad "2" smd roundrect (at 0.75 0 180) (size 0.9 0.9) (layers "F.Cu" "F.Mask" "F.Paste") (roundrect_rratio 0.25) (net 4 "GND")))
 (gr_rect (start 40 25) (end 130 160.5) (stroke (width 0.05) (type solid)) (fill no) (layer "Edge.Cuts"))
 (segment (start 93.5 72.25) (end 89.95 72.25) (width 0.25) (layer "F.Cu") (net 18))
 (segment (start 89.95 72.25) (end 89.5 71.8) (width 0.25) (layer "F.Cu") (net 18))
 (segment (start 98.5 80) (end 105 80) (width 0.25) (layer "F.Cu") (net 4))
 (segment (start 91.25 77) (end 91.5 77) (width 0.25) (layer "F.Cu") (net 4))
 (segment (start 62.75 106) (end 61 104.25) (width 0.25) (layer "F.Cu") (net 4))
 (segment (start 93.5 75) (end 93.5 73.75) (width 0.25) (layer "F.Cu") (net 4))
 (segment (start 93.5 75) (end 98.5 80) (width 0.25) (layer "F.Cu") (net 4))
 (segment (start 61 104.25) (end 61 99.25) (width 0.25) (layer "F.Cu") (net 4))
 (segment (start 61.25 93.5) (end 61.25 98) (width 0.25) (layer "F.Cu") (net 4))
 (segment (start 61.25 99) (end 61.25 98) (width 0.25) (layer "F.Cu") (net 4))
 (segment (start 91.5 77) (end 93.5 75) (width 0.25) (layer "F.Cu") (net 4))
 (segment (start 61 99.25) (end 61.25 99) (width 0.25) (layer "F.Cu") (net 4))
 (segment (start 91 75) (end 93.5 75) (width 0.25) (layer "F.Cu") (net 4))
 (segment (start 89.5 73.5) (end 91 75) (width 0.25) (layer "F.Cu") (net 4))
 (via (at 105 80) (size 0.6) (drill 0.3) (layers "F.Cu" "B.Cu") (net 4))
 (segment (start 109.44 80) (end 105 80) (width 0.25) (layer "B.Cu") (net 4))
 (segment (start 117.53 88.09) (end 109.44 80) (width 0.25) (layer "B.Cu") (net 4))
 (segment (start 87.3 75.55) (end 88.75 77) (width 0.25) (layer "F.Cu") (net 17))
 (segment (start 87.3 73.5) (end 87.3 75.55) (width 0.25) (layer "F.Cu") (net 17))
 (segment (start 88.75 77) (end 89.75 77) (width 0.25) (layer "F.Cu") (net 17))
 (segment (start 63.75 98.5) (end 65 98.5) (width 0.25) (layer "F.Cu") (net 3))
 (segment (start 66 99.5) (end 66 100.25) (width 0.25) (layer "F.Cu") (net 3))
 (segment (start 63.25 98) (end 63.75 98.5) (width 0.25) (layer "F.Cu") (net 3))
 (segment (start 62.75 93.5) (end 62.75 98) (width 0.25) (layer "F.Cu") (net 3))
 (segment (start 62.75 98) (end 63.25 98) (width 0.25) (layer "F.Cu") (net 3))
 (segment (start 65 98.5) (end 66 99.5) (width 0.25) (layer "F.Cu") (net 3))
 (segment (start 89.15 96.95) (end 89.7 96.95) (width 0.25) (layer "F.Cu") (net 5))
 (segment (start 88.7 96.5) (end 89.15 96.95) (width 0.25) (layer "F.Cu") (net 5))
 (segment (start 89.7 96.95) (end 94.25 101.5) (width 0.25) (layer "F.Cu") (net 5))
 (segment (start 109.25 103.5) (end 112.75 103.5) (width 0.25) (layer "F.Cu") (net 2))
 (segment (start 66 104.25) (end 64.25 106) (width 0.25) (layer "F.Cu") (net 19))
 (segment (start 66 101.75) (end 66 104.25) (width 0.25) (layer "F.Cu") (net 19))
 (segment (start 80.3 98.45) (end 80.3 132.5) (width 0.25) (layer "F.Cu") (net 14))
 (segment (start 80.25 89) (end 79.75 88.5) (width 0.25) (layer "F.Cu") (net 14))
 (segment (start 82.25 96.5) (end 80.25 94.5) (width 0.25) (layer "F.Cu") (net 14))
 (segment (start 85.3 96.5) (end 82.25 96.5) (width 0.25) (layer "F.Cu") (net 14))
 (segment (start 82.25 96.5) (end 80.3 98.45) (width 0.25) (layer "F.Cu") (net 14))
 (segment (start 80.25 94.5) (end 80.25 89) (width 0.25) (layer "F.Cu") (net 14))
 (segment (start 76.61 90.86) (end 49.5 90.86) (width 0.25) (layer "F.Cu") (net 14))
 (segment (start 82.25 96.5) (end 76.61 90.86) (width 0.25) (layer "F.Cu") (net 14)))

